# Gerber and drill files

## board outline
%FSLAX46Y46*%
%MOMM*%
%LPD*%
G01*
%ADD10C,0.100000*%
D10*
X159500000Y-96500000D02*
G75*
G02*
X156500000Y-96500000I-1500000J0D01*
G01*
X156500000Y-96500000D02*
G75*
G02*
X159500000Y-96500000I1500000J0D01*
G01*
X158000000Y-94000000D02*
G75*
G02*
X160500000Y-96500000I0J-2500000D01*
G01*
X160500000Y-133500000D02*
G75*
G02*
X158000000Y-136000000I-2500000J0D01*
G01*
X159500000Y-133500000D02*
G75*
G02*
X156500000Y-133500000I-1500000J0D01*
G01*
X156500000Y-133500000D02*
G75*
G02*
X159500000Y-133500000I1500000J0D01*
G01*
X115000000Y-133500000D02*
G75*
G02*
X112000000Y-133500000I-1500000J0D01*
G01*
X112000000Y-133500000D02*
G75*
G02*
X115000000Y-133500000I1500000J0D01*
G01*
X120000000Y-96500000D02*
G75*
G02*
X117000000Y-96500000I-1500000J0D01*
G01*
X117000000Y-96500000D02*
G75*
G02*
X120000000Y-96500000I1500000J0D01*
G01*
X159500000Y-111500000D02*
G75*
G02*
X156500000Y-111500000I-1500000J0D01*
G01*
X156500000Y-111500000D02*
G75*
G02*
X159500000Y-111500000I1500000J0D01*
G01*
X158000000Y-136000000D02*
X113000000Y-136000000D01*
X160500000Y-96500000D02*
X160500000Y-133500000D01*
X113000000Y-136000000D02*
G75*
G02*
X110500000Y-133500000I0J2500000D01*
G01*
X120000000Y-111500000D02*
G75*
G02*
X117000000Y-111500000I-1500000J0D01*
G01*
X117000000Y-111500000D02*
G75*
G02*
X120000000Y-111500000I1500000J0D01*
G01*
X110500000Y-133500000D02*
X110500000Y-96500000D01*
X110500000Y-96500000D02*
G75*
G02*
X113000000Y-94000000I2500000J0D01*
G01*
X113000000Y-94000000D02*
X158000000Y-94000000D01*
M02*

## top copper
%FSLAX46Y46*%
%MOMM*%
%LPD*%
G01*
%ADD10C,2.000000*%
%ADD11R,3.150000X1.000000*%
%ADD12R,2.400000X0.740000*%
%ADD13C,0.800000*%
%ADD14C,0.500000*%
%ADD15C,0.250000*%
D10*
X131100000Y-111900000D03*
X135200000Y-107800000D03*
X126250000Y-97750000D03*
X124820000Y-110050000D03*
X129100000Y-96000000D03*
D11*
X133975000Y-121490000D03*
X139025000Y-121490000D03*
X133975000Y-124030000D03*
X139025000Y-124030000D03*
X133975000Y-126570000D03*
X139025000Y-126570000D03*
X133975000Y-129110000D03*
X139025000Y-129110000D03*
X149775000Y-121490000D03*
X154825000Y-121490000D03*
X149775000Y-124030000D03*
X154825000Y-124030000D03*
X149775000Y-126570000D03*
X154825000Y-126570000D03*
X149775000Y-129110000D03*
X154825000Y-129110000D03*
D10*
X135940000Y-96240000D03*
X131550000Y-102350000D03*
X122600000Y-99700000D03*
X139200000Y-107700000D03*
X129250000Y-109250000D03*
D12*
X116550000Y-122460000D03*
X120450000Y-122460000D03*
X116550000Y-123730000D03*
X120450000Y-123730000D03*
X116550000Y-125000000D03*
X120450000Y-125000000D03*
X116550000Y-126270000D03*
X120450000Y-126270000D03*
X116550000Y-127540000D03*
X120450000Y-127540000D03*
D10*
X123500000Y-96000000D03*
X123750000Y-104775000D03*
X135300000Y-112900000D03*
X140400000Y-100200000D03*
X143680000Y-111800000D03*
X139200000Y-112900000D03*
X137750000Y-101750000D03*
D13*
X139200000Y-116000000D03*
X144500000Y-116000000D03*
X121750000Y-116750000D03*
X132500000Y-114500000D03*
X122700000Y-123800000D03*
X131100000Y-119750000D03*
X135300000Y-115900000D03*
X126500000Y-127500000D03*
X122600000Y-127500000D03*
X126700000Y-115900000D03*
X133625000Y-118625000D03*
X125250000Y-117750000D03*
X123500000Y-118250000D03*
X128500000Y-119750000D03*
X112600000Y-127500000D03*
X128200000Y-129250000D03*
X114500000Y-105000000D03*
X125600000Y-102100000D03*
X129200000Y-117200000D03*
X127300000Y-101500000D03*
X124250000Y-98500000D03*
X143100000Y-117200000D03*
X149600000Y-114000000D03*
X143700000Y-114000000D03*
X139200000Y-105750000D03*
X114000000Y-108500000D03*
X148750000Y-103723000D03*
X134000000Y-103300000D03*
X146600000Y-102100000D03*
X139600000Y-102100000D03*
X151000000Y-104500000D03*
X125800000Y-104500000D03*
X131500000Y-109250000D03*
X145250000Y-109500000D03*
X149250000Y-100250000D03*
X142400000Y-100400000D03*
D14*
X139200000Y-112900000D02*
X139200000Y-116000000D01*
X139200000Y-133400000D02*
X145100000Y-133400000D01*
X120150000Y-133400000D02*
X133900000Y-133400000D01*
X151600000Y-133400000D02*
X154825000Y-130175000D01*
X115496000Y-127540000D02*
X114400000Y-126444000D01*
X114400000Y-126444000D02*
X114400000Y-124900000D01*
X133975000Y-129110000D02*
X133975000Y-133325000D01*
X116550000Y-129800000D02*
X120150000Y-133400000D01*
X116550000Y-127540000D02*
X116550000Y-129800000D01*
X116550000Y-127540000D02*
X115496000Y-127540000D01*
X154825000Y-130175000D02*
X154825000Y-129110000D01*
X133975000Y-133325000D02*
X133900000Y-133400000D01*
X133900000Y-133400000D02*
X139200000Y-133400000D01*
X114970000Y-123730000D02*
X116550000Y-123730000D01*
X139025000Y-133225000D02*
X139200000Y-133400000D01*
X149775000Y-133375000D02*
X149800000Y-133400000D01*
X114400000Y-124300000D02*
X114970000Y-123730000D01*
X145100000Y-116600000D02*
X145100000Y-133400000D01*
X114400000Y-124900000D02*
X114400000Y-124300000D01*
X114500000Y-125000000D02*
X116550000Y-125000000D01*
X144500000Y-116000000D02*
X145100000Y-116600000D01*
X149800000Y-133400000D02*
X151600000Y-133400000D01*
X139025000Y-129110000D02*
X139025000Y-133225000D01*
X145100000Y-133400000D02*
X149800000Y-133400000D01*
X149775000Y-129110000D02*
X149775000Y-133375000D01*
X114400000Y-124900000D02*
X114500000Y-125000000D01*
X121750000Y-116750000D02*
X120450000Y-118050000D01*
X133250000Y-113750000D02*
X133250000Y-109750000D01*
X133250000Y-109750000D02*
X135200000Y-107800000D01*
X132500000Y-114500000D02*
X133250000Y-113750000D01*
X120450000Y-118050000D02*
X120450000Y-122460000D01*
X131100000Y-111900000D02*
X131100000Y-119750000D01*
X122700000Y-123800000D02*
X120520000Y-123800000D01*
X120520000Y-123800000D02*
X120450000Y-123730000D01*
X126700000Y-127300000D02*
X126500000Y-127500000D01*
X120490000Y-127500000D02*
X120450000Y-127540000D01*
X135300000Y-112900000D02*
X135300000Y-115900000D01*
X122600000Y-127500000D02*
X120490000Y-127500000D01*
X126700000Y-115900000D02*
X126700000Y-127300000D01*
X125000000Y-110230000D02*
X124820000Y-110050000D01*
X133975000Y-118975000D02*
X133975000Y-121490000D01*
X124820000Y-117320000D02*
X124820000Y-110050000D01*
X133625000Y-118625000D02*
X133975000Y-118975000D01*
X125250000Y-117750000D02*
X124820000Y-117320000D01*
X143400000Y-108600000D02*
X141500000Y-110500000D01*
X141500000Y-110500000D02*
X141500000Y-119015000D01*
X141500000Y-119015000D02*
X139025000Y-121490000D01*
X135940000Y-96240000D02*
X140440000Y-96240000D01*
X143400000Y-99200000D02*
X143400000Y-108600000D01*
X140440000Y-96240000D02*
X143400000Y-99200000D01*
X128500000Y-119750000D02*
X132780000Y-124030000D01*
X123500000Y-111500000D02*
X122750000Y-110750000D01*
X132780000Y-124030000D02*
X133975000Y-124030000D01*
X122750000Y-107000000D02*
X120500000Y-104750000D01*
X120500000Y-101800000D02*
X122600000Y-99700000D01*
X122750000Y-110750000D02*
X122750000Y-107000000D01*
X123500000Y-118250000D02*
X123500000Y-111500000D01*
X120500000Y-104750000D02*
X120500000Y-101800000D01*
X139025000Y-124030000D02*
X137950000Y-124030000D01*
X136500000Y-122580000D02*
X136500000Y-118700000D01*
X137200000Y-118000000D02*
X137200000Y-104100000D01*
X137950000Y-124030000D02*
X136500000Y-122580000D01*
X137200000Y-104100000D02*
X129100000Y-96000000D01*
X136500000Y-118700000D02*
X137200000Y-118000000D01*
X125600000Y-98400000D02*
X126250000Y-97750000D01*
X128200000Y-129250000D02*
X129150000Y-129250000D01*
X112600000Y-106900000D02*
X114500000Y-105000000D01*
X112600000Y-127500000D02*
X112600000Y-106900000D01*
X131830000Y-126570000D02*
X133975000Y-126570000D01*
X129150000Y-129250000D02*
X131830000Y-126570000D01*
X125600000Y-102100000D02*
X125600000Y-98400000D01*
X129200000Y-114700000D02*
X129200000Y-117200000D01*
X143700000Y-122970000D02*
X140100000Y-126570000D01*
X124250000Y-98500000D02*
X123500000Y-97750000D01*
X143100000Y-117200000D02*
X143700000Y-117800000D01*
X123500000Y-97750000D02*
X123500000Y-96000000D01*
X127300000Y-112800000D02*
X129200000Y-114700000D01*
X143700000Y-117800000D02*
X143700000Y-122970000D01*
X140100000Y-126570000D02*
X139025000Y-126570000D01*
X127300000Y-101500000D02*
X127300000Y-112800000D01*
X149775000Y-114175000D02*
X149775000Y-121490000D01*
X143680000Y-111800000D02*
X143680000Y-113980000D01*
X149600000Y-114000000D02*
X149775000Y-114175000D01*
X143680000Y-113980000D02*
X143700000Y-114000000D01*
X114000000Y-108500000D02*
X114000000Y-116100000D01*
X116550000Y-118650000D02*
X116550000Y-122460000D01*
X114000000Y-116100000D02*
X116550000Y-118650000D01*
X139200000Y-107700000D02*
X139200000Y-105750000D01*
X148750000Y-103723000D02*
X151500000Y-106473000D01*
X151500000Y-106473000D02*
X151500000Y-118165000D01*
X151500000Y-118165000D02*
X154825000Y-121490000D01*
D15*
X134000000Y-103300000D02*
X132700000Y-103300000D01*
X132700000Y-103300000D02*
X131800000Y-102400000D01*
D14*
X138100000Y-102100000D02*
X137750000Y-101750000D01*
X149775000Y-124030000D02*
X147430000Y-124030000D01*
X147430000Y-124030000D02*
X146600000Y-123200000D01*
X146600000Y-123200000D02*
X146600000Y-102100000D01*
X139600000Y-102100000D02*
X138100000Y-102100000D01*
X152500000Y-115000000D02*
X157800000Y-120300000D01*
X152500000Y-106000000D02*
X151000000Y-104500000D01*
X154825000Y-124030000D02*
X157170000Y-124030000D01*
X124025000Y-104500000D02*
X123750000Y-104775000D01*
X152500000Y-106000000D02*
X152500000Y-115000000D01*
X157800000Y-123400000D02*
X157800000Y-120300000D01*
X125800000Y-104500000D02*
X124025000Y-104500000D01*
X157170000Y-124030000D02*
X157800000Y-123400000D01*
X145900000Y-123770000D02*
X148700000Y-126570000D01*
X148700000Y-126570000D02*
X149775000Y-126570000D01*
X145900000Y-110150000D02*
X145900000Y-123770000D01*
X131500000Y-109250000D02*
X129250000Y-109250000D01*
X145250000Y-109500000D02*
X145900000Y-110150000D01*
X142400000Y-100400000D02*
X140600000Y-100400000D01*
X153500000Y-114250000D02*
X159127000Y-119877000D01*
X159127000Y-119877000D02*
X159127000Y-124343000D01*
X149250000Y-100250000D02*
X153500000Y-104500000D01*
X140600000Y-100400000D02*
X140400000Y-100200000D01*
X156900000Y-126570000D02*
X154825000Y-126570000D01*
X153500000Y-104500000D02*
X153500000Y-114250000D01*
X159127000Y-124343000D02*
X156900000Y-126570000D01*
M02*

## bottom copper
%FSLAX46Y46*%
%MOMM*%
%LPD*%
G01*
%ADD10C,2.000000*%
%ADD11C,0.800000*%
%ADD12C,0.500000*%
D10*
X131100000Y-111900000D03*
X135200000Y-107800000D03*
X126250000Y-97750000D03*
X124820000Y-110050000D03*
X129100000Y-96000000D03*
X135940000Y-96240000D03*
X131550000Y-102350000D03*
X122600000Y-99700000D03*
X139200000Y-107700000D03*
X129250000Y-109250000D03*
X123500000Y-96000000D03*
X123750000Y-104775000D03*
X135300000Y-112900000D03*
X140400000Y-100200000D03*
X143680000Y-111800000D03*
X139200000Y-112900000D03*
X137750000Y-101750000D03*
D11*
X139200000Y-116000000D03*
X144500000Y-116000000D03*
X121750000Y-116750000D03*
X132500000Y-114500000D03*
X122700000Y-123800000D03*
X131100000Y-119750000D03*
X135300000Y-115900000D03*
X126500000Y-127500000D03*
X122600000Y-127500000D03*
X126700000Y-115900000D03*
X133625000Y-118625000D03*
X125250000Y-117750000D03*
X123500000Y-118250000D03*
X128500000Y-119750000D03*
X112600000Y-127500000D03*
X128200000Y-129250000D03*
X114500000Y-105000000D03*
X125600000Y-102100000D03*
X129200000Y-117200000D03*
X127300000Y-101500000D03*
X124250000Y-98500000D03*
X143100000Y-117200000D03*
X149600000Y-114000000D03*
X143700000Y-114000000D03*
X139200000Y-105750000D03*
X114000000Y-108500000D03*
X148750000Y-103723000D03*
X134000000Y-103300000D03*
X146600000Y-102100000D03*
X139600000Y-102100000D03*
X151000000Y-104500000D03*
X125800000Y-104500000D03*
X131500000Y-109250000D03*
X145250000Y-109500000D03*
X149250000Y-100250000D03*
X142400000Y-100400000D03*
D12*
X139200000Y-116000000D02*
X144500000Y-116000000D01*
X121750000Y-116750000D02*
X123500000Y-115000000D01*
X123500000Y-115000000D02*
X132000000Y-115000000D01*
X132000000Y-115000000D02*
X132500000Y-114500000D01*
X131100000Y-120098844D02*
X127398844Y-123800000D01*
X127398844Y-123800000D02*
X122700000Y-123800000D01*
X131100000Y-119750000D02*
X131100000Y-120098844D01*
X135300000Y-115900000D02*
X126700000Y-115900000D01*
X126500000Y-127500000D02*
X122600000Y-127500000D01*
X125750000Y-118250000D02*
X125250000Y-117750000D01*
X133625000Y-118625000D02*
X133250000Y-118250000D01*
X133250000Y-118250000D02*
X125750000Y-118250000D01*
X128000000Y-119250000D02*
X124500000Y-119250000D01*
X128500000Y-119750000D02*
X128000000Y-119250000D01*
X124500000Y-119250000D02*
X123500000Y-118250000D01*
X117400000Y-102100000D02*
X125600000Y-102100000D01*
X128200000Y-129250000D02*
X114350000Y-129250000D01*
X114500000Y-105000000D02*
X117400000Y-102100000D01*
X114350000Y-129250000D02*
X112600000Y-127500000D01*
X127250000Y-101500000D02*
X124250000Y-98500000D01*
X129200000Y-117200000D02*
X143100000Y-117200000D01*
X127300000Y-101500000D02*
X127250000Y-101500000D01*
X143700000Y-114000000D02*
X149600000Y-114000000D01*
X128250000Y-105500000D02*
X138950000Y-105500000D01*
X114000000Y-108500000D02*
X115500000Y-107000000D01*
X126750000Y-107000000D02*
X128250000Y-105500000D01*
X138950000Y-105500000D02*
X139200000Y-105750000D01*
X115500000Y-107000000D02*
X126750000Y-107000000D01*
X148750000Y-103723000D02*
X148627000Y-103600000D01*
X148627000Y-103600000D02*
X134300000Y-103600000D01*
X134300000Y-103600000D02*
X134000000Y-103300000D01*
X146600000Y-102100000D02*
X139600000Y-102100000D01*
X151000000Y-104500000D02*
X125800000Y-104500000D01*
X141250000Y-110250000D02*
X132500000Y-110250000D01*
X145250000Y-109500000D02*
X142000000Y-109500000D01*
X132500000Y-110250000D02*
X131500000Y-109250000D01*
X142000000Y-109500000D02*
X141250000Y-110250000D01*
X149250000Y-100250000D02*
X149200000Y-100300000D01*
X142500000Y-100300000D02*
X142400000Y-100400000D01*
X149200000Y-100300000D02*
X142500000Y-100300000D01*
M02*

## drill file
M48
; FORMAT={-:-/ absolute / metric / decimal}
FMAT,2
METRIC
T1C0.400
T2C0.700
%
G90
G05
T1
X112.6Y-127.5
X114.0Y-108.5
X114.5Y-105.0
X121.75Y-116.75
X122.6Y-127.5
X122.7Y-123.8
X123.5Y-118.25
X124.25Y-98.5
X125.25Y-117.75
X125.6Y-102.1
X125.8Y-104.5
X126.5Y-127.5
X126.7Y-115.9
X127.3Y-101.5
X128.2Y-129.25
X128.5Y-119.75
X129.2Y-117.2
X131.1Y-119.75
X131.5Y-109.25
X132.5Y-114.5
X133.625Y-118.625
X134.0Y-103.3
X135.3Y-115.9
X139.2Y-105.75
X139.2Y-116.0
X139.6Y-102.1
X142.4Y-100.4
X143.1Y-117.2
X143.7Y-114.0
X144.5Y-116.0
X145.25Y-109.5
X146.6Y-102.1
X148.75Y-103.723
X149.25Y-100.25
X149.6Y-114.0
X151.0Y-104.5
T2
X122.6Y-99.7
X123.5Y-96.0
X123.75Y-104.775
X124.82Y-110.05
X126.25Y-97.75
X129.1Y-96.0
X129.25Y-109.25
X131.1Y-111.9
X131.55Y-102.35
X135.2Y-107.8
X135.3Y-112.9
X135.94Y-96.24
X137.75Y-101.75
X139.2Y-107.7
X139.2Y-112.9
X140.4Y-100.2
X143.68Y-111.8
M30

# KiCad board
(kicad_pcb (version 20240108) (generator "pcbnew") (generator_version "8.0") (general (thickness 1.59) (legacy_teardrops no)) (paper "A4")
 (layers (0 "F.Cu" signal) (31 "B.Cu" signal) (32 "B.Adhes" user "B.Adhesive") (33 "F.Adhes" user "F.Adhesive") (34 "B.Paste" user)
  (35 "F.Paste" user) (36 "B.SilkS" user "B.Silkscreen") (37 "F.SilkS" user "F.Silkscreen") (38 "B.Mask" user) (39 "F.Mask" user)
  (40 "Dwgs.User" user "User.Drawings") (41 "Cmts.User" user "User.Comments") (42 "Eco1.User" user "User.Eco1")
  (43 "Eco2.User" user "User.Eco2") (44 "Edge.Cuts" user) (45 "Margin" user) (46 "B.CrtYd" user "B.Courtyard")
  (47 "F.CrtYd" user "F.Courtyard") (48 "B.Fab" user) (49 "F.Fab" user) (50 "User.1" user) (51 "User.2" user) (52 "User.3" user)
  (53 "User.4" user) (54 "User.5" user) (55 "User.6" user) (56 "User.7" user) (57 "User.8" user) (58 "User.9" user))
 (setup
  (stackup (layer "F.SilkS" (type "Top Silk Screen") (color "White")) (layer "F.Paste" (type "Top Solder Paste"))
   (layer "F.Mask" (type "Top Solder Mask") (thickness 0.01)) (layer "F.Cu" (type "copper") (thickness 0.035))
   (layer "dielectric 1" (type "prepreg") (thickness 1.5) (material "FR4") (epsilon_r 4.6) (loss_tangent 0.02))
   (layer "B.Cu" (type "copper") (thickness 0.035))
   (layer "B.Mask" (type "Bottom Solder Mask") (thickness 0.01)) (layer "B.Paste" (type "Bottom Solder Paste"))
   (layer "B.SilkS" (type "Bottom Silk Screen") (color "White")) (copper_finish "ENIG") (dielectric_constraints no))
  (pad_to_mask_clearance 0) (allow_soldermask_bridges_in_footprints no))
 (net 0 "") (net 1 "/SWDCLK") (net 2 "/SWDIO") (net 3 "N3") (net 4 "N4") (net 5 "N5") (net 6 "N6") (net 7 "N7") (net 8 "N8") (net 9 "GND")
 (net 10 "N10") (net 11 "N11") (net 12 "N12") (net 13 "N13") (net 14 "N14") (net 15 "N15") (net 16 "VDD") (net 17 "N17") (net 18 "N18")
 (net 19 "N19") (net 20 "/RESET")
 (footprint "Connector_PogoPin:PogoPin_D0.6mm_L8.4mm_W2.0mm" (layer "F.Cu") (at 131.1 111.9)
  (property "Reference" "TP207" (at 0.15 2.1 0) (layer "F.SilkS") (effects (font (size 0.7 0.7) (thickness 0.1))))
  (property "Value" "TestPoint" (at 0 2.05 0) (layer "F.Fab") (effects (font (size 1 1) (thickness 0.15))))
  (pad "1" thru_hole circle (at 0 0) (size 2 2) (drill 0.7) (layers "*.Cu" "*.Mask") (remove_unused_layers no) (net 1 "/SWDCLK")))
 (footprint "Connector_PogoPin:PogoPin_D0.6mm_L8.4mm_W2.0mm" (layer "F.Cu") (at 135.2 107.8)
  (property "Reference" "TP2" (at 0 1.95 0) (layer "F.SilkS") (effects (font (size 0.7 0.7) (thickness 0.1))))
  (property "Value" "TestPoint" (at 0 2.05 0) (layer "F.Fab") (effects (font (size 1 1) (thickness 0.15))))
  (pad "1" thru_hole circle (at 0 0) (size 2 2) (drill 0.7) (layers "*.Cu" "*.Mask") (remove_unused_layers no) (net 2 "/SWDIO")))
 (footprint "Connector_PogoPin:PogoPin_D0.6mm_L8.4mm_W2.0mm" (layer "F.Cu") (at 126.25 97.75)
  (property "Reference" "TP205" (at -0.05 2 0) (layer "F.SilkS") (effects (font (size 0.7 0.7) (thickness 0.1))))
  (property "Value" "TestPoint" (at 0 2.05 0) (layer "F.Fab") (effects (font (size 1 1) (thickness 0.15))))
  (pad "1" thru_hole circle (at 0 0) (size 2 2) (drill 0.7) (layers "*.Cu" "*.Mask") (remove_unused_layers no) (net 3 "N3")))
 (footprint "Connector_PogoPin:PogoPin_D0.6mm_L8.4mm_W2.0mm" (layer "F.Cu") (at 124.82 110.05)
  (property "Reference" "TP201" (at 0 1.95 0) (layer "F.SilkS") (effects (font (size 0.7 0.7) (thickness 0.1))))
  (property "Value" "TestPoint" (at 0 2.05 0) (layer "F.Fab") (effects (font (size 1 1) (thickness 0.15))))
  (pad "1" thru_hole circle (at 0 0) (size 2 2) (drill 0.7) (layers "*.Cu" "*.Mask") (remove_unused_layers no) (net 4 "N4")))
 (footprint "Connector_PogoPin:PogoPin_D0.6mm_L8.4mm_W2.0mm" (layer "F.Cu") (at 129.1 96)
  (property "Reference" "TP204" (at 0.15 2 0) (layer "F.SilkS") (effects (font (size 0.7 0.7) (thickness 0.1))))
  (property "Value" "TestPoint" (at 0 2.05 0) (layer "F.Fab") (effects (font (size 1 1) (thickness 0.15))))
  (pad "1" thru_hole circle (at 0 0) (size 2 2) (drill 0.7) (layers "*.Cu" "*.Mask") (remove_unused_layers no) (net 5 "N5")))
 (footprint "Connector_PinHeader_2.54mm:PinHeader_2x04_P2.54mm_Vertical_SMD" (layer "F.Cu") (at 136.5 125.3)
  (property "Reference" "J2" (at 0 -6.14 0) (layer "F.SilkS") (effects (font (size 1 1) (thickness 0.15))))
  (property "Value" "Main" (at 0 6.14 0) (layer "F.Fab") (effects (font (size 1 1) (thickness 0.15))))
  (pad "1" smd rect (at -2.525 -3.81) (size 3.15 1) (layers "F.Cu" "F.Paste" "F.Mask") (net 4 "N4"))
  (pad "2" smd rect (at 2.525 -3.81) (size 3.15 1) (layers "F.Cu" "F.Paste" "F.Mask") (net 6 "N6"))
  (pad "3" smd rect (at -2.525 -1.27) (size 3.15 1) (layers "F.Cu" "F.Paste" "F.Mask") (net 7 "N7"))
  (pad "4" smd rect (at 2.525 -1.27) (size 3.15 1) (layers "F.Cu" "F.Paste" "F.Mask") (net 5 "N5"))
  (pad "5" smd rect (at -2.525 1.27) (size 3.15 1) (layers "F.Cu" "F.Paste" "F.Mask") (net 3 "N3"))
  (pad "6" smd rect (at 2.525 1.27) (size 3.15 1) (layers "F.Cu" "F.Paste" "F.Mask") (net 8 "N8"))
  (pad "7" smd rect (at -2.525 3.81) (size 3.15 1) (layers "F.Cu" "F.Paste" "F.Mask") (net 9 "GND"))
  (pad "8" smd rect (at 2.525 3.81) (size 3.15 1) (layers "F.Cu" "F.Paste" "F.Mask") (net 9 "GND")))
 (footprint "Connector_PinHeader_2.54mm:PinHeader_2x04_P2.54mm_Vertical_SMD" (layer "F.Cu") (at 152.3 125.3)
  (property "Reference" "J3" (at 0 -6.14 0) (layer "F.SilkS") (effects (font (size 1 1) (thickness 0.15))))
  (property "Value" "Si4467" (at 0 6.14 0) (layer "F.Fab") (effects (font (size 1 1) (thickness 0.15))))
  (pad "1" smd rect (at -2.525 -3.81) (size 3.15 1) (layers "F.Cu" "F.Paste" "F.Mask") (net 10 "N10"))
  (pad "2" smd rect (at 2.525 -3.81) (size 3.15 1) (layers "F.Cu" "F.Paste" "F.Mask") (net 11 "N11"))
  (pad "3" smd rect (at -2.525 -1.27) (size 3.15 1) (layers "F.Cu" "F.Paste" "F.Mask") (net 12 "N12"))
  (pad "4" smd rect (at 2.525 -1.27) (size 3.15 1) (layers "F.Cu" "F.Paste" "F.Mask") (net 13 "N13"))
  (pad "5" smd rect (at -2.525 1.27) (size 3.15 1) (layers "F.Cu" "F.Paste" "F.Mask") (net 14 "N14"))
  (pad "6" smd rect (at 2.525 1.27) (size 3.15 1) (layers "F.Cu" "F.Paste" "F.Mask") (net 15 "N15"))
  (pad "7" smd rect (at -2.525 3.81) (size 3.15 1) (layers "F.Cu" "F.Paste" "F.Mask") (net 9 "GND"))
  (pad "8" smd rect (at 2.525 3.81) (size 3.15 1) (layers "F.Cu" "F.Paste" "F.Mask") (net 9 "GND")))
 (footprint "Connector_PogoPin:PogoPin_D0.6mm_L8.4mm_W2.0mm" (layer "F.Cu") (at 135.94 96.24)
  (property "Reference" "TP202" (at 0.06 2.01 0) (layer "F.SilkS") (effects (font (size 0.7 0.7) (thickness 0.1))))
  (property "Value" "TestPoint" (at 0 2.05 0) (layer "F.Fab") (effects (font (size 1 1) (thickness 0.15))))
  (pad "1" thru_hole circle (at 0 0) (size 2 2) (drill 0.7) (layers "*.Cu" "*.Mask") (remove_unused_layers no) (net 6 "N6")))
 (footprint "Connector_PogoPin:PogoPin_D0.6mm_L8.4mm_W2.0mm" (layer "F.Cu") (at 131.55 102.35)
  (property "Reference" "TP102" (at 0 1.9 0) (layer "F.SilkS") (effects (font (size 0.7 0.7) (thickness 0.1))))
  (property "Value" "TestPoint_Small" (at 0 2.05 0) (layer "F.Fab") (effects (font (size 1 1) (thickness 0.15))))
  (pad "1" thru_hole circle (at 0 0) (size 2 2) (drill 0.7) (layers "*.Cu" "*.Mask") (remove_unused_layers no) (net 11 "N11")))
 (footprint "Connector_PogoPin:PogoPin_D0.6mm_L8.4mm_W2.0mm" (layer "F.Cu") (at 122.6 99.7)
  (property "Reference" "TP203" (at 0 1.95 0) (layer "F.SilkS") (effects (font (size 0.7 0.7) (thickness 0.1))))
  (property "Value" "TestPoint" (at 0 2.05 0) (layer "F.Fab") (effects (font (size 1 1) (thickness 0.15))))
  (pad "1" thru_hole circle (at 0 0) (size 2 2) (drill 0.7) (layers "*.Cu" "*.Mask") (remove_unused_layers no) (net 7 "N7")))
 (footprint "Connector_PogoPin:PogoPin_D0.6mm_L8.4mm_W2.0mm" (layer "F.Cu") (at 139.2 107.7)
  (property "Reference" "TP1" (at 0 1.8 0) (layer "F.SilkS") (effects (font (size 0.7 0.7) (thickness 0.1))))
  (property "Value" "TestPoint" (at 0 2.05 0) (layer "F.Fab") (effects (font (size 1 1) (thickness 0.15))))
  (pad "1" thru_hole circle (at 0 0) (size 2 2) (drill 0.7) (layers "*.Cu" "*.Mask") (remove_unused_layers no) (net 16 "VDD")))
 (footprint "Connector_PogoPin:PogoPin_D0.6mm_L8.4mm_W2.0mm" (layer "F.Cu") (at 129.25 109.25)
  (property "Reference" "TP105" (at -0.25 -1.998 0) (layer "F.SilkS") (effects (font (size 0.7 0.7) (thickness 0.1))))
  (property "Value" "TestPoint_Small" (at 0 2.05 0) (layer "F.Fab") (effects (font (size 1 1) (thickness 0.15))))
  (pad "1" thru_hole circle (at 0 0) (size 2 2) (drill 0.7) (layers "*.Cu" "*.Mask") (remove_unused_layers no) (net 14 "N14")))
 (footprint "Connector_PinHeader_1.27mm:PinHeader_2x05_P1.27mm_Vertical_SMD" (layer "F.Cu") (at 118.5 125)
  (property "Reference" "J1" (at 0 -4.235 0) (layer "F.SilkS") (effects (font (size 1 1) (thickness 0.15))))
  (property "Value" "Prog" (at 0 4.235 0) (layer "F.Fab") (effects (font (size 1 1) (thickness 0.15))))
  (pad "1" smd rect (at -1.95 -2.54) (size 2.4 0.74) (layers "F.Cu" "F.Paste" "F.Mask") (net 16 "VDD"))
  (pad "2" smd rect (at 1.95 -2.54) (size 2.4 0.74) (layers "F.Cu" "F.Paste" "F.Mask") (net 2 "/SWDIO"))
  (pad "3" smd rect (at -1.95 -1.27) (size 2.4 0.74) (layers "F.Cu" "F.Paste" "F.Mask") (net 9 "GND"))
  (pad "4" smd rect (at 1.95 -1.27) (size 2.4 0.74) (layers "F.Cu" "F.Paste" "F.Mask") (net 1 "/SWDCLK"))
  (pad "5" smd rect (at -1.95 0) (size 2.4 0.74) (layers "F.Cu" "F.Paste" "F.Mask") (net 9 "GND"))
  (pad "6" smd rect (at 1.95 0) (size 2.4 0.74) (layers "F.Cu" "F.Paste" "F.Mask") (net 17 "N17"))
  (pad "7" smd rect (at -1.95 1.27) (size 2.4 0.74) (layers "F.Cu" "F.Paste" "F.Mask") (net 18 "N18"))
  (pad "8" smd rect (at 1.95 1.27) (size 2.4 0.74) (layers "F.Cu" "F.Paste" "F.Mask") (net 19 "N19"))
  (pad "9" smd rect (at -1.95 2.54) (size 2.4 0.74) (layers "F.Cu" "F.Paste" "F.Mask") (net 9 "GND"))
  (pad "10" smd rect (at 1.95 2.54) (size 2.4 0.74) (layers "F.Cu" "F.Paste" "F.Mask") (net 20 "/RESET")))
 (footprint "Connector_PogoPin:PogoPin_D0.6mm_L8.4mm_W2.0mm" (layer "F.Cu") (at 123.5 96)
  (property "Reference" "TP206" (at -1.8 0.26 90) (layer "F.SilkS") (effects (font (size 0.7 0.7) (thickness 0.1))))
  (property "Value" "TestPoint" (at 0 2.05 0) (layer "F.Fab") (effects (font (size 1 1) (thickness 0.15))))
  (pad "1" thru_hole circle (at 0 0) (size 2 2) (drill 0.7) (layers "*.Cu" "*.Mask") (remove_unused_layers no) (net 8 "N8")))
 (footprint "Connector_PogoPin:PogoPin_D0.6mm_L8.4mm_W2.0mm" (layer "F.Cu") (at 123.75 104.775)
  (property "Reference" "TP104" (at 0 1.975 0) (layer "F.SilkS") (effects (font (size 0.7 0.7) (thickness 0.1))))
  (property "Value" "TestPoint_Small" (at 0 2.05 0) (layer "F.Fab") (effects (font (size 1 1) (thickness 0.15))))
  (pad "1" thru_hole circle (at 0 0) (size 2 2) (drill 0.7) (layers "*.Cu" "*.Mask") (remove_unused_layers no) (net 13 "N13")))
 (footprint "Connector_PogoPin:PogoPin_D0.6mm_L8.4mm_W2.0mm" (layer "F.Cu") (at 135.3 112.9)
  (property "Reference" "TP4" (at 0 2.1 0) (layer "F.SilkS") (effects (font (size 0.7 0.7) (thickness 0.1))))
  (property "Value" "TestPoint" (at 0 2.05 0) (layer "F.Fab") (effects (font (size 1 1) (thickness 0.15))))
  (pad "1" thru_hole circle (at 0 0) (size 2 2) (drill 0.7) (layers "*.Cu" "*.Mask") (remove_unused_layers no) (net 20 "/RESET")))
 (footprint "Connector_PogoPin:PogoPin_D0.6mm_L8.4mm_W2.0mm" (layer "F.Cu") (at 140.4 100.2)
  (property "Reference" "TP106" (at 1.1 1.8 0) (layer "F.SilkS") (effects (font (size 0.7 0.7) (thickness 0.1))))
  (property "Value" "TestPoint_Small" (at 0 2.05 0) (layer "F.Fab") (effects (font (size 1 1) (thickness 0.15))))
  (pad "1" thru_hole circle (at 0 0) (size 2 2) (drill 0.7) (layers "*.Cu" "*.Mask") (remove_unused_layers no) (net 15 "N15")))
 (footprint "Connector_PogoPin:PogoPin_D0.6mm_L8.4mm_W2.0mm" (layer "F.Cu") (at 143.68 111.8)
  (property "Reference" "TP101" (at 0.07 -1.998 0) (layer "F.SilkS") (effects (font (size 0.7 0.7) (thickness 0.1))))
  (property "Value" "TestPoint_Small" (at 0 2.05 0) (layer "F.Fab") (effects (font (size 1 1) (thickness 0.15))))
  (pad "1" thru_hole circle (at 0 0) (size 2 2) (drill 0.7) (layers "*.Cu" "*.Mask") (remove_unused_layers no) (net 10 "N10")))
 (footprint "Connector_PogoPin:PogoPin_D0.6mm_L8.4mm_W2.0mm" (layer "F.Cu") (at 139.2 112.9)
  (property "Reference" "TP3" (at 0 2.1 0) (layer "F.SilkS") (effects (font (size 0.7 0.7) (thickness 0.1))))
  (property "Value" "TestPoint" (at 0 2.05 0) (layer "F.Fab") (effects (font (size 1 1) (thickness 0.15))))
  (pad "1" thru_hole circle (at 0 0) (size 2 2) (drill 0.7) (layers "*.Cu" "*.Mask") (remove_unused_layers no) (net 9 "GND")))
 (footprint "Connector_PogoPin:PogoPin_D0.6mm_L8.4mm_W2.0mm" (layer "F.Cu") (at 137.75 101.75)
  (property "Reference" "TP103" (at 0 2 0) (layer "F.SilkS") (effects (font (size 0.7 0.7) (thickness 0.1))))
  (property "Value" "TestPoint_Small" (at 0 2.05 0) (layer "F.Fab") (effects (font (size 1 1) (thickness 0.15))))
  (pad "1" thru_hole circle (at 0 0) (size 2 2) (drill 0.7) (layers "*.Cu" "*.Mask") (remove_unused_layers no) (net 12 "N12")))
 (gr_circle (center 158 96.5) (end 159.5 96.5) (stroke (width 0.1) (type solid)) (fill none) (layer "Edge.Cuts"))
 (gr_arc (start 158 94) (mid 159.767767 94.732233) (end 160.5 96.5) (stroke (width 0.1) (type solid)) (layer "Edge.Cuts"))
 (gr_arc (start 160.5 133.5) (mid 159.767767 135.267767) (end 158 136) (stroke (width 0.1) (type solid)) (layer "Edge.Cuts"))
 (gr_circle (center 158 133.5) (end 159.5 133.5) (stroke (width 0.1) (type solid)) (fill none) (layer "Edge.Cuts"))
 (gr_circle (center 113.5 133.5) (end 112 133.5) (stroke (width 0.1) (type solid)) (fill none) (layer "Edge.Cuts"))
 (gr_circle (center 118.5 96.5) (end 117 96.5) (stroke (width 0.1) (type solid)) (fill none) (layer "Edge.Cuts"))
 (gr_circle (center 158 111.5) (end 159.5 111.5) (stroke (width 0.1) (type solid)) (fill none) (layer "Edge.Cuts"))
 (gr_line (start 158 136) (end 113 136) (stroke (width 0.1) (type solid)) (layer "Edge.Cuts"))
 (gr_line (start 160.5 96.5) (end 160.5 133.5) (stroke (width 0.1) (type solid)) (layer "Edge.Cuts"))
 (gr_arc (start 113 136) (mid 111.232233 135.267767) (end 110.5 133.5) (stroke (width 0.1) (type solid)) (layer "Edge.Cuts"))
 (gr_circle (center 118.5 111.5) (end 117 111.5) (stroke (width 0.1) (type solid)) (fill none) (layer "Edge.Cuts"))
 (gr_line (start 110.5 133.5) (end 110.5 96.5) (stroke (width 0.1) (type solid)) (layer "Edge.Cuts"))
 (gr_arc (start 110.5 96.5) (mid 111.232233 94.732233) (end 113 94) (stroke (width 0.1) (type solid)) (layer "Edge.Cuts"))
 (gr_line (start 113 94) (end 158 94) (stroke (width 0.1) (type solid)) (layer "Edge.Cuts"))
 (segment (start 139.2 112.9) (end 139.2 116) (width 0.5) (layer "F.Cu") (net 9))
 (segment (start 139.2 133.4) (end 145.1 133.4) (width 0.5) (layer "F.Cu") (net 9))
 (segment (start 120.15 133.4) (end 133.9 133.4) (width 0.5) (layer "F.Cu") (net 9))
 (segment (start 151.6 133.4) (end 154.825 130.175) (width 0.5) (layer "F.Cu") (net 9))
 (segment (start 115.496 127.54) (end 114.4 126.444) (width 0.5) (layer "F.Cu") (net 9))
 (segment (start 114.4 126.444) (end 114.4 124.9) (width 0.5) (layer "F.Cu") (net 9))
 (segment (start 133.975 129.11) (end 133.975 133.325) (width 0.5) (layer "F.Cu") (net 9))
 (segment (start 116.55 129.8) (end 120.15 133.4) (width 0.5) (layer "F.Cu") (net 9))
 (segment (start 116.55 127.54) (end 116.55 129.8) (width 0.5) (layer "F.Cu") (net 9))
 (segment (start 116.55 127.54) (end 115.496 127.54) (width 0.5) (layer "F.Cu") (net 9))
 (segment (start 154.825 130.175) (end 154.825 129.11) (width 0.5) (layer "F.Cu") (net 9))
 (segment (start 133.975 133.325) (end 133.9 133.4) (width 0.5) (layer "F.Cu") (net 9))
 (segment (start 133.9 133.4) (end 139.2 133.4) (width 0.5) (layer "F.Cu") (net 9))
 (segment (start 114.97 123.73) (end 116.55 123.73) (width 0.5) (layer "F.Cu") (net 9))
 (segment (start 139.025 133.225) (end 139.2 133.4) (width 0.5) (layer "F.Cu") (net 9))
 (segment (start 149.775 133.375) (end 149.8 133.4) (width 0.5) (layer "F.Cu") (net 9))
 (segment (start 114.4 124.3) (end 114.97 123.73) (width 0.5) (layer "F.Cu") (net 9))
 (segment (start 145.1 116.6) (end 145.1 133.4) (width 0.5) (layer "F.Cu") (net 9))
 (segment (start 114.4 124.9) (end 114.4 124.3) (width 0.5) (layer "F.Cu") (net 9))
 (segment (start 114.5 125) (end 116.55 125) (width 0.5) (layer "F.Cu") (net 9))
 (segment (start 144.5 116) (end 145.1 116.6) (width 0.5) (layer "F.Cu") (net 9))
 (segment (start 149.8 133.4) (end 151.6 133.4) (width 0.5) (layer "F.Cu") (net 9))
 (segment (start 139.025 129.11) (end 139.025 133.225) (width 0.5) (layer "F.Cu") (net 9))
 (segment (start 145.1 133.4) (end 149.8 133.4) (width 0.5) (layer "F.Cu") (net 9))
 (segment (start 149.775 129.11) (end 149.775 133.375) (width 0.5) (layer "F.Cu") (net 9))
 (segment (start 114.4 124.9) (end 114.5 125) (width 0.5) (layer "F.Cu") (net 9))
 (via (at 139.2 116) (size 0.8) (drill 0.4) (layers "F.Cu" "B.Cu") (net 9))
 (via (at 144.5 116) (size 0.8) (drill 0.4) (layers "F.Cu" "B.Cu") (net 9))
 (segment (start 139.2 116) (end 144.5 116) (width 0.5) (layer "B.Cu") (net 9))
 (segment (start 121.75 116.75) (end 120.45 118.05) (width 0.5) (layer "F.Cu") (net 2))
 (segment (start 133.25 113.75) (end 133.25 109.75) (width 0.5) (layer "F.Cu") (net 2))
 (segment (start 133.25 109.75) (end 135.2 107.8) (width 0.5) (layer "F.Cu") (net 2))
 (segment (start 132.5 114.5) (end 133.25 113.75) (width 0.5) (layer "F.Cu") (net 2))
 (segment (start 120.45 118.05) (end 120.45 122.46) (width 0.5) (layer "F.Cu") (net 2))
 (via (at 121.75 116.75) (size 0.8) (drill 0.4) (layers "F.Cu" "B.Cu") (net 2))
 (via (at 132.5 114.5) (size 0.8) (drill 0.4) (layers "F.Cu" "B.Cu") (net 2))
 (segment (start 121.75 116.75) (end 123.5 115) (width 0.5) (layer "B.Cu") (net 2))
 (segment (start 123.5 115) (end 132 115) (width 0.5) (layer "B.Cu") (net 2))
 (segment (start 132 115) (end 132.5 114.5) (width 0.5) (layer "B.Cu") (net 2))
 (segment (start 131.1 111.9) (end 131.1 119.75) (width 0.5) (layer "F.Cu") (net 1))
 (segment (start 122.7 123.8) (end 120.52 123.8) (width 0.5) (layer "F.Cu") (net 1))
 (segment (start 120.52 123.8) (end 120.45 123.73) (width 0.5) (layer "F.Cu") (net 1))
 (via (at 122.7 123.8) (size 0.8) (drill 0.4) (layers "F.Cu" "B.Cu") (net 1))
 (via (at 131.1 119.75) (size 0.8) (drill 0.4) (layers "F.Cu" "B.Cu") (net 1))
 (segment (start 131.1 120.098844) (end 127.398844 123.8) (width 0.5) (layer "B.Cu") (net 1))
 (segment (start 127.398844 123.8) (end 122.7 123.8) (width 0.5) (layer "B.Cu") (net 1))
 (segment (start 131.1 119.75) (end 131.1 120.098844) (width 0.5) (layer "B.Cu") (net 1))
 (segment (start 126.7 127.3) (end 126.5 127.5) (width 0.5) (layer "F.Cu") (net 20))
 (segment (start 120.49 127.5) (end 120.45 127.54) (width 0.5) (layer "F.Cu") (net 20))
 (segment (start 135.3 112.9) (end 135.3 115.9) (width 0.5) (layer "F.Cu") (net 20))
 (segment (start 122.6 127.5) (end 120.49 127.5) (width 0.5) (layer "F.Cu") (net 20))
 (segment (start 126.7 115.9) (end 126.7 127.3) (width 0.5) (layer "F.Cu") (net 20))
 (via (at 135.3 115.9) (size 0.8) (drill 0.4) (layers "F.Cu" "B.Cu") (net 20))
 (via (at 126.5 127.5) (size 0.8) (drill 0.4) (layers "F.Cu" "B.Cu") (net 20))
 (via (at 122.6 127.5) (size 0.8) (drill 0.4) (layers "F.Cu" "B.Cu") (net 20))
 (via (at 126.7 115.9) (size 0.8) (drill 0.4) (layers "F.Cu" "B.Cu") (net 20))
 (segment (start 135.3 115.9) (end 126.7 115.9) (width 0.5) (layer "B.Cu") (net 20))
 (segment (start 126.5 127.5) (end 122.6 127.5) (width 0.5) (layer "B.Cu") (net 20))
 (segment (start 125 110.23) (end 124.82 110.05) (width 0.5) (layer "F.Cu") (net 4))
 (segment (start 133.975 118.975) (end 133.975 121.49) (width 0.5) (layer "F.Cu") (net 4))
 (segment (start 124.82 117.32) (end 124.82 110.05) (width 0.5) (layer "F.Cu") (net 4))
 (segment (start 133.625 118.625) (end 133.975 118.975) (width 0.5) (layer "F.Cu") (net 4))
 (segment (start 125.25 117.75) (end 124.82 117.32) (width 0.5) (layer "F.Cu") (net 4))
 (via (at 133.625 118.625) (size 0.8) (drill 0.4) (layers "F.Cu" "B.Cu") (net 4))
 (via (at 125.25 117.75) (size 0.8) (drill 0.4) (layers "F.Cu" "B.Cu") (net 4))
 (segment (start 125.75 118.25) (end 125.25 117.75) (width 0.5) (layer "B.Cu") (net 4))
 (segment (start 133.625 118.625) (end 133.25 118.25) (width 0.5) (layer "B.Cu") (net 4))
 (segment (start 133.25 118.25) (end 125.75 118.25) (width 0.5) (layer "B.Cu") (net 4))
 (segment (start 143.4 108.6) (end 141.5 110.5) (width 0.5) (layer "F.Cu") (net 6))
 (segment (start 141.5 110.5) (end 141.5 119.015) (width 0.5) (layer "F.Cu") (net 6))
 (segment (start 141.5 119.015) (end 139.025 121.49) (width 0.5) (layer "F.Cu") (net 6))
 (segment (start 135.94 96.24) (end 140.44 96.24) (width 0.5) (layer "F.Cu") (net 6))
 (segment (start 143.4 99.2) (end 143.4 108.6) (width 0.5) (layer "F.Cu") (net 6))
 (segment (start 140.44 96.24) (end 143.4 99.2) (width 0.5) (layer "F.Cu") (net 6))
 (segment (start 128.5 119.75) (end 132.78 124.03) (width 0.5) (layer "F.Cu") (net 7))
 (segment (start 123.5 111.5) (end 122.75 110.75) (width 0.5) (layer "F.Cu") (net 7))
 (segment (start 132.78 124.03) (end 133.975 124.03) (width 0.5) (layer "F.Cu") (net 7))
 (segment (start 122.75 107) (end 120.5 104.75) (width 0.5) (layer "F.Cu") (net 7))
 (segment (start 120.5 101.8) (end 122.6 99.7) (width 0.5) (layer "F.Cu") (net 7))
 (segment (start 122.75 110.75) (end 122.75 107) (width 0.5) (layer "F.Cu") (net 7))
 (segment (start 123.5 118.25) (end 123.5 111.5) (width 0.5) (layer "F.Cu") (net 7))
 (segment (start 120.5 104.75) (end 120.5 101.8) (width 0.5) (layer "F.Cu") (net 7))
 (via (at 123.5 118.25) (size 0.8) (drill 0.4) (layers "F.Cu" "B.Cu") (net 7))
 (via (at 128.5 119.75) (size 0.8) (drill 0.4) (layers "F.Cu" "B.Cu") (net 7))
 (segment (start 128 119.25) (end 124.5 119.25) (width 0.5) (layer "B.Cu") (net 7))
 (segment (start 128.5 119.75) (end 128 119.25) (width 0.5) (layer "B.Cu") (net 7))
 (segment (start 124.5 119.25) (end 123.5 118.25) (width 0.5) (layer "B.Cu") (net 7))
 (segment (start 139.025 124.03) (end 137.95 124.03) (width 0.5) (layer "F.Cu") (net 5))
 (segment (start 136.5 122.58) (end 136.5 118.7) (width 0.5) (layer "F.Cu") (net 5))
 (segment (start 137.2 118) (end 137.2 104.1) (width 0.5) (layer "F.Cu") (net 5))
 (segment (start 137.95 124.03) (end 136.5 122.58) (width 0.5) (layer "F.Cu") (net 5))
 (segment (start 137.2 104.1) (end 129.1 96) (width 0.5) (layer "F.Cu") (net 5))
 (segment (start 136.5 118.7) (end 137.2 118) (width 0.5) (layer "F.Cu") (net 5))
 (segment (start 125.6 98.4) (end 126.25 97.75) (width 0.5) (layer "F.Cu") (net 3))
 (segment (start 128.2 129.25) (end 129.15 129.25) (width 0.5) (layer "F.Cu") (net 3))
 (segment (start 112.6 106.9) (end 114.5 105) (width 0.5) (layer "F.Cu") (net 3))
 (segment (start 112.6 127.5) (end 112.6 106.9) (width 0.5) (layer "F.Cu") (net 3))
 (segment (start 131.83 126.57) (end 133.975 126.57) (width 0.5) (layer "F.Cu") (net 3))
 (segment (start 129.15 129.25) (end 131.83 126.57) (width 0.5) (layer "F.Cu") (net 3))
 (segment (start 125.6 102.1) (end 125.6 98.4) (width 0.5) (layer "F.Cu") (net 3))
 (via (at 112.6 127.5) (size 0.8) (drill 0.4) (layers "F.Cu" "B.Cu") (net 3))
 (via (at 128.2 129.25) (size 0.8) (drill 0.4) (layers "F.Cu" "B.Cu") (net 3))
 (via (at 114.5 105) (size 0.8) (drill 0.4) (layers "F.Cu" "B.Cu") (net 3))
 (via (at 125.6 102.1) (size 0.8) (drill 0.4) (layers "F.Cu" "B.Cu") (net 3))
 (segment (start 117.4 102.1) (end 125.6 102.1) (width 0.5) (layer "B.Cu") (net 3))
 (segment (start 128.2 129.25) (end 114.35 129.25) (width 0.5) (layer "B.Cu") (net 3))
 (segment (start 114.5 105) (end 117.4 102.1) (width 0.5) (layer "B.Cu") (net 3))
 (segment (start 114.35 129.25) (end 112.6 127.5) (width 0.5) (layer "B.Cu") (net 3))
 (segment (start 129.2 114.7) (end 129.2 117.2) (width 0.5) (layer "F.Cu") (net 8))
 (segment (start 143.7 122.97) (end 140.1 126.57) (width 0.5) (layer "F.Cu") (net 8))
 (segment (start 124.25 98.5) (end 123.5 97.75) (width 0.5) (layer "F.Cu") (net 8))
 (segment (start 143.1 117.2) (end 143.7 117.8) (width 0.5) (layer "F.Cu") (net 8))
 (segment (start 123.5 97.75) (end 123.5 96) (width 0.5) (layer "F.Cu") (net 8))
 (segment (start 127.3 112.8) (end 129.2 114.7) (width 0.5) (layer "F.Cu") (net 8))
 (segment (start 143.7 117.8) (end 143.7 122.97) (width 0.5) (layer "F.Cu") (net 8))
 (segment (start 140.1 126.57) (end 139.025 126.57) (width 0.5) (layer "F.Cu") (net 8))
 (segment (start 127.3 101.5) (end 127.3 112.8) (width 0.5) (layer "F.Cu") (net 8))
 (via (at 129.2 117.2) (size 0.8) (drill 0.4) (layers "F.Cu" "B.Cu") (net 8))
 (via (at 127.3 101.5) (size 0.8) (drill 0.4) (layers "F.Cu" "B.Cu") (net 8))
 (via (at 124.25 98.5) (size 0.8) (drill 0.4) (layers "F.Cu" "B.Cu") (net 8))
 (via (at 143.1 117.2) (size 0.8) (drill 0.4) (layers "F.Cu" "B.Cu") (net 8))
 (segment (start 127.25 101.5) (end 124.25 98.5) (width 0.5) (layer "B.Cu") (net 8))
 (segment (start 129.2 117.2) (end 143.1 117.2) (width 0.5) (layer "B.Cu") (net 8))
 (segment (start 127.3 101.5) (end 127.25 101.5) (width 0.5) (layer "B.Cu") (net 8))
 (segment (start 149.775 114.175) (end 149.775 121.49) (width 0.5) (layer "F.Cu") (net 10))
 (segment (start 143.68 111.8) (end 143.68 113.98) (width 0.5) (layer "F.Cu") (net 10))
 (segment (start 149.6 114) (end 149.775 114.175) (width 0.5) (layer "F.Cu") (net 10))
 (segment (start 143.68 113.98) (end 143.7 114) (width 0.5) (layer "F.Cu") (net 10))
 (via (at 149.6 114) (size 0.8) (drill 0.4) (layers "F.Cu" "B.Cu") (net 10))
 (via (at 143.7 114) (size 0.8) (drill 0.4) (layers "F.Cu" "B.Cu") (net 10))
 (segment (start 143.7 114) (end 149.6 114) (width 0.5) (layer "B.Cu") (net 10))
 (segment (start 114 108.5) (end 114 116.1) (width 0.5) (layer "F.Cu") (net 16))
 (segment (start 116.55 118.65) (end 116.55 122.46) (width 0.5) (layer "F.Cu") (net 16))
 (segment (start 114 116.1) (end 116.55 118.65) (width 0.5) (layer "F.Cu") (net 16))
 (segment (start 139.2 107.7) (end 139.2 105.75) (width 0.5) (layer "F.Cu") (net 16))
 (via (at 139.2 105.75) (size 0.8) (drill 0.4) (layers "F.Cu" "B.Cu") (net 16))
 (via (at 114 108.5) (size 0.8) (drill 0.4) (layers "F.Cu" "B.Cu") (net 16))
 (segment (start 128.25 105.5) (end 138.95 105.5) (width 0.5) (layer "B.Cu") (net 16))
 (segment (start 114 108.5) (end 115.5 107) (width 0.5) (layer "B.Cu") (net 16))
 (segment (start 126.75 107) (end 128.25 105.5) (width 0.5) (layer "B.Cu") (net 16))
 (segment (start 138.95 105.5) (end 139.2 105.75) (width 0.5) (layer "B.Cu") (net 16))
 (segment (start 115.5 107) (end 126.75 107) (width 0.5) (layer "B.Cu") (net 16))
 (segment (start 148.75 103.723) (end 151.5 106.473) (width 0.5) (layer "F.Cu") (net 11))
 (segment (start 151.5 106.473) (end 151.5 118.165) (width 0.5) (layer "F.Cu") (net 11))
 (segment (start 151.5 118.165) (end 154.825 121.49) (width 0.5) (layer "F.Cu") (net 11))
 (segment (start 134 103.3) (end 132.7 103.3) (width 0.25) (layer "F.Cu") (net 11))
 (segment (start 132.7 103.3) (end 131.8 102.4) (width 0.25) (layer "F.Cu") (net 11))
 (via (at 148.75 103.723) (size 0.8) (drill 0.4) (layers "F.Cu" "B.Cu") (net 11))
 (via (at 134 103.3) (size 0.8) (drill 0.4) (layers "F.Cu" "B.Cu") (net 11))
 (segment (start 148.75 103.723) (end 148.627 103.6) (width 0.5) (layer "B.Cu") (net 11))
 (segment (start 148.627 103.6) (end 134.3 103.6) (width 0.5) (layer "B.Cu") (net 11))
 (segment (start 134.3 103.6) (end 134 103.3) (width 0.5) (layer "B.Cu") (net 11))
 (segment (start 138.1 102.1) (end 137.75 101.75) (width 0.5) (layer "F.Cu") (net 12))
 (segment (start 149.775 124.03) (end 147.43 124.03) (width 0.5) (layer "F.Cu") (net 12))
 (segment (start 147.43 124.03) (end 146.6 123.2) (width 0.5) (layer "F.Cu") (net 12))
 (segment (start 146.6 123.2) (end 146.6 102.1) (width 0.5) (layer "F.Cu") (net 12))
 (segment (start 139.6 102.1) (end 138.1 102.1) (width 0.5) (layer "F.Cu") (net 12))
 (via (at 146.6 102.1) (size 0.8) (drill 0.4) (layers "F.Cu" "B.Cu") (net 12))
 (via (at 139.6 102.1) (size 0.8) (drill 0.4) (layers "F.Cu" "B.Cu") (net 12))
 (segment (start 146.6 102.1) (end 139.6 102.1) (width 0.5) (layer "B.Cu") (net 12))
 (segment (start 152.5 115) (end 157.8 120.3) (width 0.5) (layer "F.Cu") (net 13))
 (segment (start 152.5 106) (end 151 104.5) (width 0.5) (layer "F.Cu") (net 13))
 (segment (start 154.825 124.03) (end 157.17 124.03) (width 0.5) (layer "F.Cu") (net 13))
 (segment (start 124.025 104.5) (end 123.75 104.775) (width 0.5) (layer "F.Cu") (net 13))
 (segment (start 152.5 106) (end 152.5 115) (width 0.5) (layer "F.Cu") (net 13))
 (segment (start 157.8 123.4) (end 157.8 120.3) (width 0.5) (layer "F.Cu") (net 13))
 (segment (start 125.8 104.5) (end 124.025 104.5) (width 0.5) (layer "F.Cu") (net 13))
 (segment (start 157.17 124.03) (end 157.8 123.4) (width 0.5) (layer "F.Cu") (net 13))
 (via (at 151 104.5) (size 0.8) (drill 0.4) (layers "F.Cu" "B.Cu") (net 13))
 (via (at 125.8 104.5) (size 0.8) (drill 0.4) (layers "F.Cu" "B.Cu") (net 13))
 (segment (start 151 104.5) (end 125.8 104.5) (width 0.5) (layer "B.Cu") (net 13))
 (segment (start 145.9 123.77) (end 148.7 126.57) (width 0.5) (layer "F.Cu") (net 14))
 (segment (start 148.7 126.57) (end 149.775 126.57) (width 0.5) (layer "F.Cu") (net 14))
 (segment (start 145.9 110.15) (end 145.9 123.77) (width 0.5) (layer "F.Cu") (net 14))
 (segment (start 131.5 109.25) (end 129.25 109.25) (width 0.5) (layer "F.Cu") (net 14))
 (segment (start 145.25 109.5) (end 145.9 110.15) (width 0.5) (layer "F.Cu") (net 14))
 (via (at 131.5 109.25) (size 0.8) (drill 0.4) (layers "F.Cu" "B.Cu") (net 14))
 (via (at 145.25 109.5) (size 0.8) (drill 0.4) (layers "F.Cu" "B.Cu") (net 14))
 (segment (start 141.25 110.25) (end 132.5 110.25) (width 0.5) (layer "B.Cu") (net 14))
 (segment (start 145.25 109.5) (end 142 109.5) (width 0.5) (layer "B.Cu") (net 14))
 (segment (start 132.5 110.25) (end 131.5 109.25) (width 0.5) (layer "B.Cu") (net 14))
 (segment (start 142 109.5) (end 141.25 110.25) (width 0.5) (layer "B.Cu") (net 14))
 (segment (start 142.4 100.4) (end 140.6 100.4) (width 0.5) (layer "F.Cu") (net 15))
 (segment (start 153.5 114.25) (end 159.127 119.877) (width 0.5) (layer "F.Cu") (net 15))
 (segment (start 159.127 119.877) (end 159.127 124.343) (width 0.5) (layer "F.Cu") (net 15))
 (segment (start 149.25 100.25) (end 153.5 104.5) (width 0.5) (layer "F.Cu") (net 15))
 (segment (start 140.6 100.4) (end 140.4 100.2) (width 0.5) (layer "F.Cu") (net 15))
 (segment (start 156.9 126.57) (end 154.825 126.57) (width 0.5) (layer "F.Cu") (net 15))
 (segment (start 153.5 104.5) (end 153.5 114.25) (width 0.5) (layer "F.Cu") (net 15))
 (segment (start 159.127 124.343) (end 156.9 126.57) (width 0.5) (layer "F.Cu") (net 15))
 (via (at 149.25 100.25) (size 0.8) (drill 0.4) (layers "F.Cu" "B.Cu") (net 15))
 (via (at 142.4 100.4) (size 0.8) (drill 0.4) (layers "F.Cu" "B.Cu") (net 15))
 (segment (start 149.25 100.25) (end 149.2 100.3) (width 0.5) (layer "B.Cu") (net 15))
 (segment (start 142.5 100.3) (end 142.4 100.4) (width 0.5) (layer "B.Cu") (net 15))
 (segment (start 149.2 100.3) (end 142.5 100.3) (width 0.5) (layer "B.Cu") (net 15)))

